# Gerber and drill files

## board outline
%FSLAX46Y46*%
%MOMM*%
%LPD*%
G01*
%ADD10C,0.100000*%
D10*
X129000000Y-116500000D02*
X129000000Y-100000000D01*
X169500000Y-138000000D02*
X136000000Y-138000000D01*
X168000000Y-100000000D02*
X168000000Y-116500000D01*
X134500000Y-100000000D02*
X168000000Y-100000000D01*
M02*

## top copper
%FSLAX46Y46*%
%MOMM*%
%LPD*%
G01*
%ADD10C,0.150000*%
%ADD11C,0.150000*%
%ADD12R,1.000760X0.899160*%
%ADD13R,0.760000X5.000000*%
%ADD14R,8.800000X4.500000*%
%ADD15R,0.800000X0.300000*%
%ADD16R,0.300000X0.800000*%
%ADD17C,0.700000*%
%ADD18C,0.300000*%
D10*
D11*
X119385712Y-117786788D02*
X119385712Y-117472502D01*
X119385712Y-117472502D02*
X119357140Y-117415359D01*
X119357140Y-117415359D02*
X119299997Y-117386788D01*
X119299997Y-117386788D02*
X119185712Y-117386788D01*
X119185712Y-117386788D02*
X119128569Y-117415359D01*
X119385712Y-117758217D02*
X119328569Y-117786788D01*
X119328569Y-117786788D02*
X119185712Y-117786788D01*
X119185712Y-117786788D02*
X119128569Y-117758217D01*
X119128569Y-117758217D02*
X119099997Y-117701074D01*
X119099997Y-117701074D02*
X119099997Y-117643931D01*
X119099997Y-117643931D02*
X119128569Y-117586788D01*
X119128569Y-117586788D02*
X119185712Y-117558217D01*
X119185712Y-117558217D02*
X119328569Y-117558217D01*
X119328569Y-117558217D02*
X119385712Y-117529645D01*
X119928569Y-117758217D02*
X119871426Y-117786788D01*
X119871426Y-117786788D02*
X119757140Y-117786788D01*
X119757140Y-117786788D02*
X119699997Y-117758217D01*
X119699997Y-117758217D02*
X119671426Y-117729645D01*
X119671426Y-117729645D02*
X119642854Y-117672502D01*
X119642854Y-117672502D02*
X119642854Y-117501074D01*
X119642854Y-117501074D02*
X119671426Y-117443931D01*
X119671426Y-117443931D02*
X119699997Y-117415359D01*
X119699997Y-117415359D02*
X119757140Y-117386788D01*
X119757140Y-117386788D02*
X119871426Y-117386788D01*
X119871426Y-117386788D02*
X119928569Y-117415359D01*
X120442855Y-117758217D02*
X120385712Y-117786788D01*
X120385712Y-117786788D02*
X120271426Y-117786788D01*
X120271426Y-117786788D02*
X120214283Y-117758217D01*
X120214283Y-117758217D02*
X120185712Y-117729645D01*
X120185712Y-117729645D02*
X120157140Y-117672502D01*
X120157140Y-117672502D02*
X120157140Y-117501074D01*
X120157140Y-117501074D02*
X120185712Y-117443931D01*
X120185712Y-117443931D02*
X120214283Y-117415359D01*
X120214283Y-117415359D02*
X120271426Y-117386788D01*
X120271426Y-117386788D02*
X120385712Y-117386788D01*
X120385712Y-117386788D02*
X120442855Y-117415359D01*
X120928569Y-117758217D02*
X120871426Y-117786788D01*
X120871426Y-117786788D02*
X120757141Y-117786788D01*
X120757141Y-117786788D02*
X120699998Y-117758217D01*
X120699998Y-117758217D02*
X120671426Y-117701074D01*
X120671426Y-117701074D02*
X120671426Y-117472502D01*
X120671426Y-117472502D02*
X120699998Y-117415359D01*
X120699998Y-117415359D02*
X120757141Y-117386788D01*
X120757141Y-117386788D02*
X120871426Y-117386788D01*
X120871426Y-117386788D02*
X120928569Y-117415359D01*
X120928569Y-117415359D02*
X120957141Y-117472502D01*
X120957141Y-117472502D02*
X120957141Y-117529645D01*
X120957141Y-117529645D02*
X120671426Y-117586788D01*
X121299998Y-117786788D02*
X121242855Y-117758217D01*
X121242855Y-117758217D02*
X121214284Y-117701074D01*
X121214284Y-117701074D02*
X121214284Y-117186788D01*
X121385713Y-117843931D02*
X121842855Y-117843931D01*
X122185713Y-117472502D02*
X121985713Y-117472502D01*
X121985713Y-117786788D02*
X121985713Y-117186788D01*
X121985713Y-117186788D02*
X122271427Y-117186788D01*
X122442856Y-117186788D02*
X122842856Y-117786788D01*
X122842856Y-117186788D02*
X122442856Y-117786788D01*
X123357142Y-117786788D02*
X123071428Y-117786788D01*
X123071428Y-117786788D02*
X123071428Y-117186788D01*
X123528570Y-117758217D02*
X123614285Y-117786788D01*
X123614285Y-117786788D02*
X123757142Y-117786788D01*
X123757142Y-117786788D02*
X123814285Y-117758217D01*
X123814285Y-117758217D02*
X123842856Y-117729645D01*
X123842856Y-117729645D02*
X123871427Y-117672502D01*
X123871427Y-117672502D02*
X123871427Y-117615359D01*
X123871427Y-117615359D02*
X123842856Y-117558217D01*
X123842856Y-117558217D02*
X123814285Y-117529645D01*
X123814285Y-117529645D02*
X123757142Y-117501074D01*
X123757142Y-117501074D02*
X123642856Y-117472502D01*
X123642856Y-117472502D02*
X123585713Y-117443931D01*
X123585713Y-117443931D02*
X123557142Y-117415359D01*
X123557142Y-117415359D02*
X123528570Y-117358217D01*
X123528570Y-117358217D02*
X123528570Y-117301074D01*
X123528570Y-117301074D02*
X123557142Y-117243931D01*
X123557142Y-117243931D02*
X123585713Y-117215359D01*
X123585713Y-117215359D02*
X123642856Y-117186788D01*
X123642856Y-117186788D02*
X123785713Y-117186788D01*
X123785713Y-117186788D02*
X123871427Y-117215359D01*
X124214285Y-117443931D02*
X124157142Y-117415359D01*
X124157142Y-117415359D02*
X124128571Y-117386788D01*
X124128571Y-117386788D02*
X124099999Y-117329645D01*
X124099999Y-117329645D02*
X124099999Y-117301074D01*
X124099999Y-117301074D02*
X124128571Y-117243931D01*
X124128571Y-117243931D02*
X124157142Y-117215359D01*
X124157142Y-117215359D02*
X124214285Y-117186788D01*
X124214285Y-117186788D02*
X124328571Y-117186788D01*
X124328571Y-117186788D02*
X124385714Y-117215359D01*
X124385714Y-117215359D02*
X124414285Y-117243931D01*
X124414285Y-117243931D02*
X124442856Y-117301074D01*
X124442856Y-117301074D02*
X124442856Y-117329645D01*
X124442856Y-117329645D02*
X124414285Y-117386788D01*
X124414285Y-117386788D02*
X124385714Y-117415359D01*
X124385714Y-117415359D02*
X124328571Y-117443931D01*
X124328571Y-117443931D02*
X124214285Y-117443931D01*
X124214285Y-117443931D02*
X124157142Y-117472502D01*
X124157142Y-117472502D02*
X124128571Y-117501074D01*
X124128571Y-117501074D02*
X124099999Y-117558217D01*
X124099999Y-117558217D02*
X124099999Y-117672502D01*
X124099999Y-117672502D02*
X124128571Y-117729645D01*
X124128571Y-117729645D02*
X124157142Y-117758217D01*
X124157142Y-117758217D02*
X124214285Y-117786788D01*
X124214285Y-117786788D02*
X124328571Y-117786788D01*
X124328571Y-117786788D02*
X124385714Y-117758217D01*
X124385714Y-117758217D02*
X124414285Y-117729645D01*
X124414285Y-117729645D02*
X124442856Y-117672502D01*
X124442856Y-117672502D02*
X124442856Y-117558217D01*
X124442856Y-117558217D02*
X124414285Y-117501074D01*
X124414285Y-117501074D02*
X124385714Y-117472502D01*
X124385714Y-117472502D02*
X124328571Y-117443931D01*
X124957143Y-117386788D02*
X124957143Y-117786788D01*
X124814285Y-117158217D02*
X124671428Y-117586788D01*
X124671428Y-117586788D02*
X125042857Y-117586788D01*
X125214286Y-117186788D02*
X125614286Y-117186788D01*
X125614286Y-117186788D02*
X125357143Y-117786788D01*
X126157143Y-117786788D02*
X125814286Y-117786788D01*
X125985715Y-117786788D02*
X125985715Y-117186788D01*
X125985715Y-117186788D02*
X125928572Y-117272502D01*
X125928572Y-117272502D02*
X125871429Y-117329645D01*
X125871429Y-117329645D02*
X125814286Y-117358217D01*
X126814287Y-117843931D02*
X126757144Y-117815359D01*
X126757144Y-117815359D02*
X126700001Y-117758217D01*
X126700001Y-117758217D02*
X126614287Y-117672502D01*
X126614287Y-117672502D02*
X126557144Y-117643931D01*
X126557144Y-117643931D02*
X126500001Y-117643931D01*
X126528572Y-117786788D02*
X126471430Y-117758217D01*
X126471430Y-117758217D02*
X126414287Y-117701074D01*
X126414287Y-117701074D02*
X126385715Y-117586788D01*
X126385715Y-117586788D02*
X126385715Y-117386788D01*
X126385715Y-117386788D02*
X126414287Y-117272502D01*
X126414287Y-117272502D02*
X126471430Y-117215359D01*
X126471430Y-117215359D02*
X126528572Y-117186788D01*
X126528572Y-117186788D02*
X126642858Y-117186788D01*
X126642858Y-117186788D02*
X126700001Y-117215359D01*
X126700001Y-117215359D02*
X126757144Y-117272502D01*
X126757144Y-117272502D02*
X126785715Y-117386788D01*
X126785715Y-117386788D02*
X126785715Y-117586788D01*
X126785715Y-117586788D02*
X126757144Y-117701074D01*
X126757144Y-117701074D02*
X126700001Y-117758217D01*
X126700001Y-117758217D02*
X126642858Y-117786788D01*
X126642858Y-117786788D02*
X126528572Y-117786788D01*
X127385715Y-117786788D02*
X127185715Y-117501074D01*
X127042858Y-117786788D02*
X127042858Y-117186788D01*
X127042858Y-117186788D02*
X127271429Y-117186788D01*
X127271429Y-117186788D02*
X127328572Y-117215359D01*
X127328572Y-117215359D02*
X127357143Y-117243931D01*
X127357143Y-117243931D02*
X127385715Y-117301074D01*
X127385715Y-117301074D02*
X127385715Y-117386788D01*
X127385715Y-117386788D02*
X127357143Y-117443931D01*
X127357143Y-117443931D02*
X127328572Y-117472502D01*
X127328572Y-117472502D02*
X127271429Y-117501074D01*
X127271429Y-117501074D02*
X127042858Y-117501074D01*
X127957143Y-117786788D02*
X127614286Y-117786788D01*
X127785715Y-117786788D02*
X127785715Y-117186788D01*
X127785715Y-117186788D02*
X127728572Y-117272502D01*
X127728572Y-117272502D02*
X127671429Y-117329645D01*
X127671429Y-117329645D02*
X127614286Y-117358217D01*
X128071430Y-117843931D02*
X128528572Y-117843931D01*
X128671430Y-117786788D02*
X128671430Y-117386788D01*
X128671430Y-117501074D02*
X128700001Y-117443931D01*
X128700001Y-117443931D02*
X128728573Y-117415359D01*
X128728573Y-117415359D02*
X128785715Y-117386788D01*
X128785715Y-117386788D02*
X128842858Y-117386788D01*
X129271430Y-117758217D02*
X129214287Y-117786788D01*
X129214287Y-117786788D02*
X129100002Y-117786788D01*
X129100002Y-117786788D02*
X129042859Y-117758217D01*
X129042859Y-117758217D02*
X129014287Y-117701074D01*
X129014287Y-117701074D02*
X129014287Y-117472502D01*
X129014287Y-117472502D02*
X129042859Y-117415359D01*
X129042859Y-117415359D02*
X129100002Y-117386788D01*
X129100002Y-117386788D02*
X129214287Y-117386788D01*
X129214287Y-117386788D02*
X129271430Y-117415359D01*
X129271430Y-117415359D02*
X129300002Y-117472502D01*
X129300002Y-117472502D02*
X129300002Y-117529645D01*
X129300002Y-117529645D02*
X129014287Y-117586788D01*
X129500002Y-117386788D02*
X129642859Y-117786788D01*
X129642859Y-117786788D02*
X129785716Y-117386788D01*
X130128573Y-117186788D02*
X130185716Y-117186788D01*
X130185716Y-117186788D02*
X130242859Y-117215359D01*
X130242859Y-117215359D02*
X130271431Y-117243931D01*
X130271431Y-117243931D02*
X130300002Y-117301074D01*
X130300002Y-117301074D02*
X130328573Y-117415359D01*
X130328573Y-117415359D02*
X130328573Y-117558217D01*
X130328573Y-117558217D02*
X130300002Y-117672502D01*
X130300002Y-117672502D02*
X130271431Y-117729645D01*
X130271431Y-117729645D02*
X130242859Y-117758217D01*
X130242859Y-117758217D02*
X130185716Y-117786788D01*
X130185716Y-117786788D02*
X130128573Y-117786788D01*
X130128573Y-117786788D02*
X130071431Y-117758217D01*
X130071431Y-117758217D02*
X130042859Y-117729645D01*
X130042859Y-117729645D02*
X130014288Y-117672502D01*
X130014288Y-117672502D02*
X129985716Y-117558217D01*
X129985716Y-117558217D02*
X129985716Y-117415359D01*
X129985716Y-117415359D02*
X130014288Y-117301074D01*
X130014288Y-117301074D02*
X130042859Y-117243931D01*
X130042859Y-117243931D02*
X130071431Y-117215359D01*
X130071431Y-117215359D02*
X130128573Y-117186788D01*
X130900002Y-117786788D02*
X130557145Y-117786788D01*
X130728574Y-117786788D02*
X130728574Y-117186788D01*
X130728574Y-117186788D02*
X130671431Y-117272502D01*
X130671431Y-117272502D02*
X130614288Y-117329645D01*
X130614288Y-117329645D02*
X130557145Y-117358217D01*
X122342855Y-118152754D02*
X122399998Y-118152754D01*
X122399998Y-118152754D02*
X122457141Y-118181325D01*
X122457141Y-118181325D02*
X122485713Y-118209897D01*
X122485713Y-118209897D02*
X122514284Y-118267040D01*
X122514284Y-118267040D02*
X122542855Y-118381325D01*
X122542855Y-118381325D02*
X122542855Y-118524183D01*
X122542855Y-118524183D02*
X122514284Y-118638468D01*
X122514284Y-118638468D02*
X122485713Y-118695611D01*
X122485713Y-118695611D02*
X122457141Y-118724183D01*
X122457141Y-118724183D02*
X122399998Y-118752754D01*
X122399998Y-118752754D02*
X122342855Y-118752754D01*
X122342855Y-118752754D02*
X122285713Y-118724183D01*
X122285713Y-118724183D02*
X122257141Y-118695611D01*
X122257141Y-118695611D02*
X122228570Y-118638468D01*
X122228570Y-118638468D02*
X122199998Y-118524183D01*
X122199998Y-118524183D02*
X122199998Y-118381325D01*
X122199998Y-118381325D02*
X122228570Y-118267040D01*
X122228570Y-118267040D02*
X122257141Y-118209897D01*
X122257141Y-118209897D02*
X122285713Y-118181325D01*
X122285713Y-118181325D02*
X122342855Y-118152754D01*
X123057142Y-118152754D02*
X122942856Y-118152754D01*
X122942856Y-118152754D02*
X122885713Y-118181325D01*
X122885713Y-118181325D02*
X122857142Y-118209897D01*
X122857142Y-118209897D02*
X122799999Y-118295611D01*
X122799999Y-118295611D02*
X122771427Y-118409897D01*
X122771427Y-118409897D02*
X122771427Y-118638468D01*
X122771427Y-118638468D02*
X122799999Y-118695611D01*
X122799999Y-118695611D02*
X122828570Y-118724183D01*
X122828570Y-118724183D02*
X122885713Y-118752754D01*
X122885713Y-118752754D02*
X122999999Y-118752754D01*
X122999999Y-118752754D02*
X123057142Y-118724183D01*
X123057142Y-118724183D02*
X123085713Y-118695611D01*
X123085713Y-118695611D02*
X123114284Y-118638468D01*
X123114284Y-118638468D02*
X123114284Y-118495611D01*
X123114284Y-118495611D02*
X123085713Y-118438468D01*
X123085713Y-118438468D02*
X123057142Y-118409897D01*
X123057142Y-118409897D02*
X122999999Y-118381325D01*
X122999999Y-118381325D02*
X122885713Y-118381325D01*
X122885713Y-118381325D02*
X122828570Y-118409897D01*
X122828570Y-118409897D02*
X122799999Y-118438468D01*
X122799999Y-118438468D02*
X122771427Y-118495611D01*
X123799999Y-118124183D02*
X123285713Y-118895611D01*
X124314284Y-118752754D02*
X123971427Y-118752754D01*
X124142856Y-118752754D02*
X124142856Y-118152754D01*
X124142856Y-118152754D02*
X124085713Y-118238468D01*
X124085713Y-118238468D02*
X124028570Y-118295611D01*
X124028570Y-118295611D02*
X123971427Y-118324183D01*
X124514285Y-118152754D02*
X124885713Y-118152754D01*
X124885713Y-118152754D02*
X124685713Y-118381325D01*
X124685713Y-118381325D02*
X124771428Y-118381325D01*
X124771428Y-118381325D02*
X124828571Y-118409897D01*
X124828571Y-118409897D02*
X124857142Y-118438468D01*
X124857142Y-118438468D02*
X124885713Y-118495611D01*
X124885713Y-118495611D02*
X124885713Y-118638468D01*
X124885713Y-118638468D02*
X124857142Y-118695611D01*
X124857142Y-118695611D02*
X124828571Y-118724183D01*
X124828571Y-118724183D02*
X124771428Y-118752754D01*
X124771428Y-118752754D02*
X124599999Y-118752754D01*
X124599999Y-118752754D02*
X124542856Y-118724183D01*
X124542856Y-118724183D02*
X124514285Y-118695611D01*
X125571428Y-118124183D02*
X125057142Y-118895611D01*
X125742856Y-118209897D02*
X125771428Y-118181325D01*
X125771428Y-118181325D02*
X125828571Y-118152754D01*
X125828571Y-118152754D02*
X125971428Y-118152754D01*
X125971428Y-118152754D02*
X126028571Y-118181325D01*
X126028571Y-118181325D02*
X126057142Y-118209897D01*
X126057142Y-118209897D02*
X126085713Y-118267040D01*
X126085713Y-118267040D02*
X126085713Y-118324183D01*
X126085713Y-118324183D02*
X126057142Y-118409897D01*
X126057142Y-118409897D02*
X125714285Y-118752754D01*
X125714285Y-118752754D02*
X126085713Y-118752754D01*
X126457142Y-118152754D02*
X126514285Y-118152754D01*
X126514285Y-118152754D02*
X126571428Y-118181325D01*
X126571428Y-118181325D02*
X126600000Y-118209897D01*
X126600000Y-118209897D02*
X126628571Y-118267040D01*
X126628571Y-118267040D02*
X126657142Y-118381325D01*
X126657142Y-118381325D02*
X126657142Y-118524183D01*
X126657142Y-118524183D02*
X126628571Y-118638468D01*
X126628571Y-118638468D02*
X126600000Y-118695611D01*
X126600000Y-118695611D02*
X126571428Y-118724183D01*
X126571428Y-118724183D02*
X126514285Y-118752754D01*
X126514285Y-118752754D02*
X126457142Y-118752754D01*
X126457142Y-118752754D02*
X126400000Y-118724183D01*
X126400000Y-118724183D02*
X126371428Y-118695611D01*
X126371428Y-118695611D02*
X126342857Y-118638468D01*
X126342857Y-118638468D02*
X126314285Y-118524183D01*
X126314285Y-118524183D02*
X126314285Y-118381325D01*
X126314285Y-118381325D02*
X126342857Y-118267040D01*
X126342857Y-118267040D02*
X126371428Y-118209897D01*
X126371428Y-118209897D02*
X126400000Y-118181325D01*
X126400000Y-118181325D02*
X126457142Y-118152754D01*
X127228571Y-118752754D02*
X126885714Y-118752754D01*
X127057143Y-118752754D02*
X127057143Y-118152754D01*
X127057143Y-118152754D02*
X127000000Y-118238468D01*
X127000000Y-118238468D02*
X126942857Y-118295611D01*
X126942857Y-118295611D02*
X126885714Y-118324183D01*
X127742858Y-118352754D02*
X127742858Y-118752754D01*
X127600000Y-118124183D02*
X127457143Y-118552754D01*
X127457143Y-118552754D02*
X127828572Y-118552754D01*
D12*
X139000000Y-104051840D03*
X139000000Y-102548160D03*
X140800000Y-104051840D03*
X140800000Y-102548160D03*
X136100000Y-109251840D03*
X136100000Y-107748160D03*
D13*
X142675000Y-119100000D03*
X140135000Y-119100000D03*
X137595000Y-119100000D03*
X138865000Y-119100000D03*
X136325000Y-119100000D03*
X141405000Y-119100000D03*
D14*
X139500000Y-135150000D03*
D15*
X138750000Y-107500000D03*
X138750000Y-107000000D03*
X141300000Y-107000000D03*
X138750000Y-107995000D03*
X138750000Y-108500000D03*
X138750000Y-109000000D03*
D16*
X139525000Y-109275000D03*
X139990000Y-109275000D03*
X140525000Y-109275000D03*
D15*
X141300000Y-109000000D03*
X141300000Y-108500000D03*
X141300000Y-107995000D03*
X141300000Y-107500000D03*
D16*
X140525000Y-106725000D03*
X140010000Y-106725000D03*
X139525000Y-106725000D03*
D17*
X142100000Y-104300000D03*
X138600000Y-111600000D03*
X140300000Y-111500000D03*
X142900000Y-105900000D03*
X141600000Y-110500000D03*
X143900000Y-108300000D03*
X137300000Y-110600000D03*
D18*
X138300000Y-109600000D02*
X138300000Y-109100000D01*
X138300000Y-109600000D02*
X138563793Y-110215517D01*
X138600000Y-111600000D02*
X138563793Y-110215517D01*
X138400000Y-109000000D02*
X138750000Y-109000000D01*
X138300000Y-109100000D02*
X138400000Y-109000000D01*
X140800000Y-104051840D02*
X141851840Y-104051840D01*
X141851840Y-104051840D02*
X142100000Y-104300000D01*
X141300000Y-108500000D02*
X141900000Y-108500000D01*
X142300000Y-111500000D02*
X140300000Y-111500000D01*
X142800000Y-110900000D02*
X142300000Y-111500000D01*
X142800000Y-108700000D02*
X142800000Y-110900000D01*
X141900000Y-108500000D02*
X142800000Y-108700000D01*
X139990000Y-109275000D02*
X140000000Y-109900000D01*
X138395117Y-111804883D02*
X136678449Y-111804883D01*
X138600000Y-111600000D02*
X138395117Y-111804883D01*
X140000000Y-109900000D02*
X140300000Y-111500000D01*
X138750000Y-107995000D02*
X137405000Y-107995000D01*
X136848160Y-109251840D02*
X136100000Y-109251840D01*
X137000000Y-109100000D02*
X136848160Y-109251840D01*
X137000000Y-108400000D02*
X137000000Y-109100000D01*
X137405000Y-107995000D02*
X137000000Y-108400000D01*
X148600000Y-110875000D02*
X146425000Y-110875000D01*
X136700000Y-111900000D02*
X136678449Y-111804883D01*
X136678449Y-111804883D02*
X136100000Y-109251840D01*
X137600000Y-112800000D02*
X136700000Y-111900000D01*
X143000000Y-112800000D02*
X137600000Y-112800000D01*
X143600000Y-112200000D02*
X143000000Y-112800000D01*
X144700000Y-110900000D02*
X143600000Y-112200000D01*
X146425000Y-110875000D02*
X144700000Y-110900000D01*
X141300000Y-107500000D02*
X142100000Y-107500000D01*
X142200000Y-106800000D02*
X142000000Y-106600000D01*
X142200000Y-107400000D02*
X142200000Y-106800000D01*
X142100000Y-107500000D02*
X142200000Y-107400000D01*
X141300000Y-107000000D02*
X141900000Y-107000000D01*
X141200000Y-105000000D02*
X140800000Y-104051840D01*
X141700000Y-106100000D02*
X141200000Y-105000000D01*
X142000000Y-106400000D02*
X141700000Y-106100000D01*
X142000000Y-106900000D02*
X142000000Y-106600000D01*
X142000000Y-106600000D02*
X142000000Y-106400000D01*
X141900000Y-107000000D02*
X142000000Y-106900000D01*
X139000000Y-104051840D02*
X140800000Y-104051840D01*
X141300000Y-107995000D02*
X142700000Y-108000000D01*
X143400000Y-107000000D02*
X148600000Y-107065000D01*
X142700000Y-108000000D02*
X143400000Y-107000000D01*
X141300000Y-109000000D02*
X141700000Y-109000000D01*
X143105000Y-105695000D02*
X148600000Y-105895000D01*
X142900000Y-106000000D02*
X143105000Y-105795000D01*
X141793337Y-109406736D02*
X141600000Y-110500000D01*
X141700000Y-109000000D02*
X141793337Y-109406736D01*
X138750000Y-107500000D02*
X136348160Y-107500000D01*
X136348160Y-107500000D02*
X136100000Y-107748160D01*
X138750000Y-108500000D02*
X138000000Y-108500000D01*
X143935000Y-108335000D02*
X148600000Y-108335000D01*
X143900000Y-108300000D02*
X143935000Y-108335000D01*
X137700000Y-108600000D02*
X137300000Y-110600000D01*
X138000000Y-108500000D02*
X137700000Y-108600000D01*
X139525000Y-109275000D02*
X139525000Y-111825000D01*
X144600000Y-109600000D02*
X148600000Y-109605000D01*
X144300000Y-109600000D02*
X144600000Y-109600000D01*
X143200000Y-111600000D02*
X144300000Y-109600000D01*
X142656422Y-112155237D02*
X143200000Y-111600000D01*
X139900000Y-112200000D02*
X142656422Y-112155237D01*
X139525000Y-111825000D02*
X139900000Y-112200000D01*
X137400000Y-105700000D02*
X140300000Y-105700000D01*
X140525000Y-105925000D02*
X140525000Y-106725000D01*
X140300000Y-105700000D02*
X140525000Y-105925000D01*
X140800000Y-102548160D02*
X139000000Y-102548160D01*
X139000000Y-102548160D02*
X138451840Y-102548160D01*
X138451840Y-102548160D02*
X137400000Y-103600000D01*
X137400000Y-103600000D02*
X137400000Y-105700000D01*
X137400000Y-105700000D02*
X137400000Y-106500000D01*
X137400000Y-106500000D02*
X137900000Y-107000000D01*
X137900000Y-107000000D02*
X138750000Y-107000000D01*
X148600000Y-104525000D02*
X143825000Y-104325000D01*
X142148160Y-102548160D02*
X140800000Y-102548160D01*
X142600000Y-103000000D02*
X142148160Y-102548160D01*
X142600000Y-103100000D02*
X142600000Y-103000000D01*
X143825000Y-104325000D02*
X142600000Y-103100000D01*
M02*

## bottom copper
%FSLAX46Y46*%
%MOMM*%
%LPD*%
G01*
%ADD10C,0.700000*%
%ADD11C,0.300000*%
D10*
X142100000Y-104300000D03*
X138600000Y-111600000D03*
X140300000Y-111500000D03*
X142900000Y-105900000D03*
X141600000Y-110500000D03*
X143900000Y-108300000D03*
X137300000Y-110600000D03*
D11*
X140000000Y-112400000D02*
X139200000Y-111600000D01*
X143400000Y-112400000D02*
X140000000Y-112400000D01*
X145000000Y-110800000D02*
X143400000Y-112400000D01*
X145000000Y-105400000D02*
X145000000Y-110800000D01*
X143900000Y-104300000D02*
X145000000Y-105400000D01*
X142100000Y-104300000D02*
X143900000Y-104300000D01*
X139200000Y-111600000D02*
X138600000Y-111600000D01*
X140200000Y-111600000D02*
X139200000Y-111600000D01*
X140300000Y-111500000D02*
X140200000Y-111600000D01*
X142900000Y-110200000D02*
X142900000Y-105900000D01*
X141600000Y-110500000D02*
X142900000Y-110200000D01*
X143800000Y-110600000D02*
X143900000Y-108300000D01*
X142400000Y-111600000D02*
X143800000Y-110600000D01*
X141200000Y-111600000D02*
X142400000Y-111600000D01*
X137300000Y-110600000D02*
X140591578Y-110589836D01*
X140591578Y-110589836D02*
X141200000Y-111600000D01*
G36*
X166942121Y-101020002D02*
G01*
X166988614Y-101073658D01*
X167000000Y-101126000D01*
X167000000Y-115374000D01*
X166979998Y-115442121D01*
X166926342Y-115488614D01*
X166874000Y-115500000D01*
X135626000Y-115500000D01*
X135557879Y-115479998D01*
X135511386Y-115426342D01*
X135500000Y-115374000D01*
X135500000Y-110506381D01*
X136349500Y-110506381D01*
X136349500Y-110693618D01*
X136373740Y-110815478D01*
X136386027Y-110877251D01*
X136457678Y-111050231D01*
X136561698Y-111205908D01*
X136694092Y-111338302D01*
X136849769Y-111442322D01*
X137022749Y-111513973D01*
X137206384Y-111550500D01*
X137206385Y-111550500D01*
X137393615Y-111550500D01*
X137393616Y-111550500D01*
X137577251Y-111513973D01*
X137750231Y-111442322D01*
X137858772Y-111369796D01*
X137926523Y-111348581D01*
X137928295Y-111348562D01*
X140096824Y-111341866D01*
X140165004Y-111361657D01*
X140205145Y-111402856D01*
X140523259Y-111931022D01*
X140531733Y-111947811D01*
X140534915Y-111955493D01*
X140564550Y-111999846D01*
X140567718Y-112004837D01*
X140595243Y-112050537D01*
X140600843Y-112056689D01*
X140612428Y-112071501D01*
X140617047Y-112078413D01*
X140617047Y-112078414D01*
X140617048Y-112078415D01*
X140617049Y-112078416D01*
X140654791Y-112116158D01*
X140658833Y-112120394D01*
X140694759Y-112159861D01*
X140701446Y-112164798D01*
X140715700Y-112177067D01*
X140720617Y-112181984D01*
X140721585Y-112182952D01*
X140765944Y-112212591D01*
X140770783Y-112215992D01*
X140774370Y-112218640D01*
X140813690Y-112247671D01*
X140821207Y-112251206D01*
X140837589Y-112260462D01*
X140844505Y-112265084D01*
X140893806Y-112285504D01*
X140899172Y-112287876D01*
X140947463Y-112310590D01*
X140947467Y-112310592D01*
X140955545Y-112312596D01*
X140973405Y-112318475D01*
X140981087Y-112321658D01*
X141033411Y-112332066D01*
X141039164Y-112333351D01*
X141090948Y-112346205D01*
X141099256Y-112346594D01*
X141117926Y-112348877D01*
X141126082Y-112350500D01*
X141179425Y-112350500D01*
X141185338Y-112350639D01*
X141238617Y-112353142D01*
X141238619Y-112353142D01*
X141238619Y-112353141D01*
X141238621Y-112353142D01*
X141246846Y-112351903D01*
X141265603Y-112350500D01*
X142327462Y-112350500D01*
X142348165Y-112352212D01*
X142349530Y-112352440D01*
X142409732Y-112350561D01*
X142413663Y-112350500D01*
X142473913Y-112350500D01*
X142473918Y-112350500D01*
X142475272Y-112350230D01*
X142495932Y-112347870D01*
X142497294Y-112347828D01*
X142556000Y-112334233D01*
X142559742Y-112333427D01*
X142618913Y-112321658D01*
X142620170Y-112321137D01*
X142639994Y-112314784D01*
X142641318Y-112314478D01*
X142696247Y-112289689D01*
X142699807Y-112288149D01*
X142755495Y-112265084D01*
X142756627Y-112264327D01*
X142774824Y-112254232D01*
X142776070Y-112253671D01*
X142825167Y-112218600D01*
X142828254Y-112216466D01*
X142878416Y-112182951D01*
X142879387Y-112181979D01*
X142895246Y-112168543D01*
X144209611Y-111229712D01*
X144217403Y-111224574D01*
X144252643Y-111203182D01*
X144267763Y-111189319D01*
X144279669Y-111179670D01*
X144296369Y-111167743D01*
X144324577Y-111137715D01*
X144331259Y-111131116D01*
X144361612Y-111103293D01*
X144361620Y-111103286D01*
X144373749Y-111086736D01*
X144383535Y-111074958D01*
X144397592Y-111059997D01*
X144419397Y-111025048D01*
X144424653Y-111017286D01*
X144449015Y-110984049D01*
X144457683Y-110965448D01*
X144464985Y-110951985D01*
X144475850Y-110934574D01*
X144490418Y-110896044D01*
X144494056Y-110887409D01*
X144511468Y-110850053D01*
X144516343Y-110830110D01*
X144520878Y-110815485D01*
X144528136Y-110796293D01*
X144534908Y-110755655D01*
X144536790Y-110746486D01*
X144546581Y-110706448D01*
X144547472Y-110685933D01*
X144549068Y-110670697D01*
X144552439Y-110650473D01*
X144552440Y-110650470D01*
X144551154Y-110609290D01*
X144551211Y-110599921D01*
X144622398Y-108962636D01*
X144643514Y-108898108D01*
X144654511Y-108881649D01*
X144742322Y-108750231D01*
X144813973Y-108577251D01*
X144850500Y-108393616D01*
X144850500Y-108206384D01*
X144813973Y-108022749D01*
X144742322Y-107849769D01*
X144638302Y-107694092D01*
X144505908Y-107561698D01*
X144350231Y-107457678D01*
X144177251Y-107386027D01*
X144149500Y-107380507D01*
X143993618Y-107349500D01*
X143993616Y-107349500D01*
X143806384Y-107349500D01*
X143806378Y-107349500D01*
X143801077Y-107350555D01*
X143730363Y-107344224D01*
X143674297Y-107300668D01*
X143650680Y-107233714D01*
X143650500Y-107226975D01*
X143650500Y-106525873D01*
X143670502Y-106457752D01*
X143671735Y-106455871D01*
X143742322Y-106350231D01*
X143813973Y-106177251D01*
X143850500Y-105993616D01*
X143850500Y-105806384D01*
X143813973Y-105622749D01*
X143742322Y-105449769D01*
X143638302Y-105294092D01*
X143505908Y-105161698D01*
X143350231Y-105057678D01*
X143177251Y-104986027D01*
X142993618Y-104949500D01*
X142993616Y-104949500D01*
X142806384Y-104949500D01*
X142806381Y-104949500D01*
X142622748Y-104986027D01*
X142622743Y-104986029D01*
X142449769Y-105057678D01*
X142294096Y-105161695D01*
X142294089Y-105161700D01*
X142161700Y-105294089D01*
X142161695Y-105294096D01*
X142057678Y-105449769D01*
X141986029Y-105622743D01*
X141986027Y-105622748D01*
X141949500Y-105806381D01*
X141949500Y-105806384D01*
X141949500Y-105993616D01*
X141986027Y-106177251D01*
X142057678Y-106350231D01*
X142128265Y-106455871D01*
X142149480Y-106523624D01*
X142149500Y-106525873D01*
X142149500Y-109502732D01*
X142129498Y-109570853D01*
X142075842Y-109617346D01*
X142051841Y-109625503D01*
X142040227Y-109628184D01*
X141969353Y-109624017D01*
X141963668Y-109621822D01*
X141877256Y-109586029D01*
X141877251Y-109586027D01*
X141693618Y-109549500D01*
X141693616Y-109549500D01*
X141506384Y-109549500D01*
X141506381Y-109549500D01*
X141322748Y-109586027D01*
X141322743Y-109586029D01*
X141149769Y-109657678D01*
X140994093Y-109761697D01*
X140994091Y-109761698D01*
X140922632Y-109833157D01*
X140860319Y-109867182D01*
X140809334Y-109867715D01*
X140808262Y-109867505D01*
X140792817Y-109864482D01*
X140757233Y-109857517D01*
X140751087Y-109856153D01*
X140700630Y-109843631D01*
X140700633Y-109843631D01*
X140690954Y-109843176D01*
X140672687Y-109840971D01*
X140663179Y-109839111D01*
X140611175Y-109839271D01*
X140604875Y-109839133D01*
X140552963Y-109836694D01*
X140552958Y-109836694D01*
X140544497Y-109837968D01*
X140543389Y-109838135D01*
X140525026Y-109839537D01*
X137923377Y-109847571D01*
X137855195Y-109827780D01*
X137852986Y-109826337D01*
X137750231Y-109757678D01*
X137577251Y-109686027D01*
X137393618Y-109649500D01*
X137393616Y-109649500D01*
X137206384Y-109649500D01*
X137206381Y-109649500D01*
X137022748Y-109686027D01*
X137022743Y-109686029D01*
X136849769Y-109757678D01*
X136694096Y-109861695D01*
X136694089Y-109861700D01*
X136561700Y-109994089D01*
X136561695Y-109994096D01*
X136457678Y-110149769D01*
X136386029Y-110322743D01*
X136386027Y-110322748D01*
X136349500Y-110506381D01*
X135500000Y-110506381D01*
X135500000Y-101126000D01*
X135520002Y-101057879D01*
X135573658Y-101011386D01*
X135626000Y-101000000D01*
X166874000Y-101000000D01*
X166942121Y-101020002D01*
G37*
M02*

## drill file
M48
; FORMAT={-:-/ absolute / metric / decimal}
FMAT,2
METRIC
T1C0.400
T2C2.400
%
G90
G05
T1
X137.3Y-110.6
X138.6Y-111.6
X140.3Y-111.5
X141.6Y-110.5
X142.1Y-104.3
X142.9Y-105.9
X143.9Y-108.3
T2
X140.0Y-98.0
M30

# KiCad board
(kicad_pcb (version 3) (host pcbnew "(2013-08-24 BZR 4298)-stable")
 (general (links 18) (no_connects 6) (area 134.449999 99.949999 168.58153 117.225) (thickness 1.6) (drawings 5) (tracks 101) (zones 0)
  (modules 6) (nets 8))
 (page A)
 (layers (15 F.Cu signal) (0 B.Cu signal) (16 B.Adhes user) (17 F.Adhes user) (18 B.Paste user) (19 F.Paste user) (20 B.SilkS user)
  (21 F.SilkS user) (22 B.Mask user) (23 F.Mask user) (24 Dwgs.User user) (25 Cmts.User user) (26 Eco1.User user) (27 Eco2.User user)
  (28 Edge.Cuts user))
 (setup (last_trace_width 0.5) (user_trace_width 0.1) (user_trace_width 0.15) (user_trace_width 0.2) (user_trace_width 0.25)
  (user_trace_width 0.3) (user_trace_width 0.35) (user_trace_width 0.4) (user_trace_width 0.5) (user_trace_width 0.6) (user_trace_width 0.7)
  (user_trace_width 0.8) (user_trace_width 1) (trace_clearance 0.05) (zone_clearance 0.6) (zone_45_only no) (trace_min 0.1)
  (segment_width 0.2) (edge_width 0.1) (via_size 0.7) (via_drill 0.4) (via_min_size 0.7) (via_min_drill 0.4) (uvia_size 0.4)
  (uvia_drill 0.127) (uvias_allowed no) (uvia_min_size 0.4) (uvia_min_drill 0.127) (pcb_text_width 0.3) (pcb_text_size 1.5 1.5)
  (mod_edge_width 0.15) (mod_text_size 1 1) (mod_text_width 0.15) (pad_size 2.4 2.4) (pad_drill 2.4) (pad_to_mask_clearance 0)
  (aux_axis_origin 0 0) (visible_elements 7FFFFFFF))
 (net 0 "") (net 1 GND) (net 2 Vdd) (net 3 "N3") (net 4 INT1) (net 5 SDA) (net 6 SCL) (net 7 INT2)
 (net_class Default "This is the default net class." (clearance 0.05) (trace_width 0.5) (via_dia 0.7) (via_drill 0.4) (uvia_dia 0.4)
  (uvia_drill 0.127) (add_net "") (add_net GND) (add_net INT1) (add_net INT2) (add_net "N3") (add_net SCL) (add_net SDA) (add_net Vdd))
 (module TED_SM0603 (layer F.Cu) (at 139 103.3 270)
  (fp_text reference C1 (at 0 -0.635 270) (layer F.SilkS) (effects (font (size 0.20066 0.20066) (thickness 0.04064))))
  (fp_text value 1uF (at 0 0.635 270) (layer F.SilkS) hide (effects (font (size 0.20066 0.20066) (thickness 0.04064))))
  (pad 2 smd rect (at 0.75184 0 270) (size 0.89916 1.00076) (layers F.Cu F.Paste F.Mask) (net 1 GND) (clearance 0.1))
  (pad 1 smd rect (at -0.75184 0 270) (size 0.89916 1.00076) (layers F.Cu F.Paste F.Mask) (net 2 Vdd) (clearance 0.1)))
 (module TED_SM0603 (layer F.Cu) (at 140.8 103.3 270)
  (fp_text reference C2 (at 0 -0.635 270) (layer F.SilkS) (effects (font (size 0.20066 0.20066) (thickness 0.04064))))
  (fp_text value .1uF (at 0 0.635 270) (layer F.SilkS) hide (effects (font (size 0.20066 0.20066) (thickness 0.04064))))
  (pad 2 smd rect (at 0.75184 0 270) (size 0.89916 1.00076) (layers F.Cu F.Paste F.Mask) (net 1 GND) (clearance 0.1))
  (pad 1 smd rect (at -0.75184 0 270) (size 0.89916 1.00076) (layers F.Cu F.Paste F.Mask) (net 2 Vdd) (clearance 0.1)))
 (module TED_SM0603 (layer F.Cu) (at 136.1 108.5 270)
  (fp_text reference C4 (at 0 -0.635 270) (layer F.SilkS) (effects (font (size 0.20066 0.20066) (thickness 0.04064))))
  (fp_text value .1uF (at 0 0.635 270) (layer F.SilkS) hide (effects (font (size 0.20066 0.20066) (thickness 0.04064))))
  (pad 2 smd rect (at 0.75184 0 270) (size 0.89916 1.00076) (layers F.Cu F.Paste F.Mask) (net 1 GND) (clearance 0.1))
  (pad 1 smd rect (at -0.75184 0 270) (size 0.89916 1.00076) (layers F.Cu F.Paste F.Mask) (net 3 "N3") (clearance 0.1)))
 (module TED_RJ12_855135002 (layer F.Cu) (at 139.5 127 180)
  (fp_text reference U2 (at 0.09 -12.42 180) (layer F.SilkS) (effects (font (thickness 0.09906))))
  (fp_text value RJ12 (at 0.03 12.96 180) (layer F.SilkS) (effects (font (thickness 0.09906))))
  (pad 6 smd rect (at -3.175 7.9 180) (size 0.76 5) (layers F.Cu F.Paste F.Mask) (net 2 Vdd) (clearance 0.2))
  (pad 4 smd rect (at -0.635 7.9 180) (size 0.76 5) (layers F.Cu F.Paste F.Mask) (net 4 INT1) (clearance 0.2))
  (pad 2 smd rect (at 1.905 7.9 180) (size 0.76 5) (layers F.Cu F.Paste F.Mask) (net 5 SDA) (clearance 0.2))
  (pad 3 smd rect (at 0.635 7.9 180) (size 0.76 5) (layers F.Cu F.Paste F.Mask) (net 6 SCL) (clearance 0.2))
  (pad 1 smd rect (at 3.175 7.9 180) (size 0.76 5) (layers F.Cu F.Paste F.Mask) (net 1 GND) (clearance 0.2))
  (pad 5 smd rect (at -1.905 7.9 180) (size 0.76 5) (layers F.Cu F.Paste F.Mask) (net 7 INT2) (clearance 0.2))
  (pad PAD smd rect (at 0 -8.15 180) (size 8.8 4.5) (layers F.Cu F.Paste F.Mask)))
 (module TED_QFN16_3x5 (layer F.Cu) (at 140.025 108) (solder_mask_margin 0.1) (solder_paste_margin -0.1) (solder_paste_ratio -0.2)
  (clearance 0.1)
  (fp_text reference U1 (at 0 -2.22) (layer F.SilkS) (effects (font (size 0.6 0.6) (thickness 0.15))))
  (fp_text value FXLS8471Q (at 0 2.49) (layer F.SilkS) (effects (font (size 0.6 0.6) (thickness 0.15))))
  (pad 2 smd rect (at -1.275 -0.5) (size 0.8 0.3) (layers F.Cu F.Paste F.Mask) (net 3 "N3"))
  (pad 1 smd rect (at -1.275 -1) (size 0.8 0.3) (layers F.Cu F.Paste F.Mask) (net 2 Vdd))
  (pad 13 smd rect (at 1.275 -1) (size 0.8 0.3) (layers F.Cu F.Paste F.Mask) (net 1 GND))
  (pad 3 smd rect (at -1.275 -0.005) (size 0.8 0.3) (layers F.Cu F.Paste F.Mask) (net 1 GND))
  (pad 4 smd rect (at -1.275 0.5) (size 0.8 0.3) (layers F.Cu F.Paste F.Mask) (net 6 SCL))
  (pad 5 smd rect (at -1.275 1) (size 0.8 0.3) (layers F.Cu F.Paste F.Mask) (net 1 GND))
  (pad 6 smd rect (at -0.5 1.275) (size 0.3 0.8) (layers F.Cu F.Paste F.Mask) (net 5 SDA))
  (pad 7 smd rect (at -0.035 1.275) (size 0.3 0.8) (layers F.Cu F.Paste F.Mask) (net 1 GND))
  (pad 8 smd rect (at 0.5 1.275) (size 0.3 0.8) (layers F.Cu F.Paste F.Mask))
  (pad 9 smd rect (at 1.275 1) (size 0.8 0.3) (layers F.Cu F.Paste F.Mask) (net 7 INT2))
  (pad 10 smd rect (at 1.275 0.5) (size 0.8 0.3) (layers F.Cu F.Paste F.Mask) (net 1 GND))
  (pad 11 smd rect (at 1.275 -0.005) (size 0.8 0.3) (layers F.Cu F.Paste F.Mask) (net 4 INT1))
  (pad 12 smd rect (at 1.275 -0.5) (size 0.8 0.3) (layers F.Cu F.Paste F.Mask) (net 1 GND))
  (pad 14 smd rect (at 0.5 -1.275) (size 0.3 0.8) (layers F.Cu F.Paste F.Mask) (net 2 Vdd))
  (pad 15 smd rect (at -0.015 -1.275) (size 0.3 0.8) (layers F.Cu F.Paste F.Mask))
  (pad 16 smd rect (at -0.5 -1.275) (size 0.3 0.8) (layers F.Cu F.Paste F.Mask)))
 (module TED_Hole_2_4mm (layer F.Cu) (at 132.5 108)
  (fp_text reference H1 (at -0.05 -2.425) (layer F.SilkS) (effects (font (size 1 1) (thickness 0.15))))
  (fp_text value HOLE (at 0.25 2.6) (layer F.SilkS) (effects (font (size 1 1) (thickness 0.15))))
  (pad "" np_thru_hole circle (at 7.5 -10) (size 2.4 2.4) (drill 2.4) (layers *.Cu *.Mask F.SilkS)))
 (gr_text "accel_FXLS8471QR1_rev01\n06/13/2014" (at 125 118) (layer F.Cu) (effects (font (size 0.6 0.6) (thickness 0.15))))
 (gr_line (start 129 116.5) (end 129 100) (angle 90) (layer Edge.Cuts) (width 0.1))
 (gr_line (start 169.5 138) (end 136 138) (angle 90) (layer Edge.Cuts) (width 0.1))
 (gr_line (start 168 100) (end 168 116.5) (angle 90) (layer Edge.Cuts) (width 0.1))
 (gr_line (start 134.5 100) (end 168 100) (angle 90) (layer Edge.Cuts) (width 0.1))
 (segment (start 138.3 109.6) (end 138.3 109.1) (width 0.3) (layer F.Cu) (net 1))
 (segment (start 138.3 109.6) (end 138.563793 110.215517) (width 0.3) (layer F.Cu) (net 1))
 (segment (start 138.6 111.6) (end 138.563793 110.215517) (width 0.3) (layer F.Cu) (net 1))
 (segment (start 138.4 109) (end 138.75 109) (width 0.3) (layer F.Cu) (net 1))
 (segment (start 138.3 109.1) (end 138.4 109) (width 0.3) (layer F.Cu) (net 1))
 (segment (start 140.8 104.05184) (end 141.85184 104.05184) (width 0.3) (layer F.Cu) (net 1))
 (segment (start 140 112.4) (end 139.2 111.6) (width 0.3) (layer B.Cu) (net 1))
 (segment (start 143.4 112.4) (end 140 112.4) (width 0.3) (layer B.Cu) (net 1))
 (segment (start 145 110.8) (end 143.4 112.4) (width 0.3) (layer B.Cu) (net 1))
 (segment (start 145 105.4) (end 145 110.8) (width 0.3) (layer B.Cu) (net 1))
 (segment (start 143.9 104.3) (end 145 105.4) (width 0.3) (layer B.Cu) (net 1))
 (segment (start 142.1 104.3) (end 143.9 104.3) (width 0.3) (layer B.Cu) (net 1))
 (via (at 142.1 104.3) (size 0.7) (layers F.Cu B.Cu) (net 1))
 (segment (start 141.85184 104.05184) (end 142.1 104.3) (width 0.3) (layer F.Cu) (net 1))
 (segment (start 141.3 108.5) (end 141.9 108.5) (width 0.3) (layer F.Cu) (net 1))
 (segment (start 142.3 111.5) (end 140.3 111.5) (width 0.3) (layer F.Cu) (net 1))
 (segment (start 142.8 110.9) (end 142.3 111.5) (width 0.3) (layer F.Cu) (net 1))
 (segment (start 142.8 108.7) (end 142.8 110.9) (width 0.3) (layer F.Cu) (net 1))
 (segment (start 141.9 108.5) (end 142.8 108.7) (width 0.3) (layer F.Cu) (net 1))
 (segment (start 139.99 109.275) (end 140 109.9) (width 0.3) (layer F.Cu) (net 1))
 (segment (start 138.395117 111.804883) (end 136.678449 111.804883) (width 0.3) (layer F.Cu) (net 1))
 (segment (start 138.6 111.6) (end 138.395117 111.804883) (width 0.3) (layer F.Cu) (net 1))
 (via (at 138.6 111.6) (size 0.7) (layers F.Cu B.Cu) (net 1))
 (segment (start 139.2 111.6) (end 138.6 111.6) (width 0.3) (layer B.Cu) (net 1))
 (segment (start 140.2 111.6) (end 139.2 111.6) (width 0.3) (layer B.Cu) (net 1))
 (via (at 140.3 111.5) (size 0.7) (layers F.Cu B.Cu) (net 1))
 (segment (start 140.3 111.5) (end 140.2 111.6) (width 0.3) (layer B.Cu) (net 1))
 (segment (start 140 109.9) (end 140.3 111.5) (width 0.3) (layer F.Cu) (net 1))
 (segment (start 138.75 107.995) (end 137.405 107.995) (width 0.3) (layer F.Cu) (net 1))
 (segment (start 136.84816 109.25184) (end 136.1 109.25184) (width 0.3) (layer F.Cu) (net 1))
 (segment (start 137 109.1) (end 136.84816 109.25184) (width 0.3) (layer F.Cu) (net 1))
 (segment (start 137 108.4) (end 137 109.1) (width 0.3) (layer F.Cu) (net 1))
 (segment (start 137.405 107.995) (end 137 108.4) (width 0.3) (layer F.Cu) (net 1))
 (segment (start 148.6 110.875) (end 146.425 110.875) (width 0.3) (layer F.Cu) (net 1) (status 30))
 (segment (start 136.7 111.9) (end 136.678449 111.804883) (width 0.3) (layer F.Cu) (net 1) (status 20))
 (segment (start 136.678449 111.804883) (end 136.1 109.25184) (width 0.3) (layer F.Cu) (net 1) (status 20))
 (segment (start 137.6 112.8) (end 136.7 111.9) (width 0.3) (layer F.Cu) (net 1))
 (segment (start 143 112.8) (end 137.6 112.8) (width 0.3) (layer F.Cu) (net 1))
 (segment (start 143.6 112.2) (end 143 112.8) (width 0.3) (layer F.Cu) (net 1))
 (segment (start 144.7 110.9) (end 143.6 112.2) (width 0.3) (layer F.Cu) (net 1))
 (segment (start 146.425 110.875) (end 144.7 110.9) (width 0.3) (layer F.Cu) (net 1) (status 10))
 (segment (start 141.3 107.5) (end 142.1 107.5) (width 0.3) (layer F.Cu) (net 1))
 (segment (start 142.2 106.8) (end 142 106.6) (width 0.3) (layer F.Cu) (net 1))
 (segment (start 142.2 107.4) (end 142.2 106.8) (width 0.3) (layer F.Cu) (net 1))
 (segment (start 142.1 107.5) (end 142.2 107.4) (width 0.3) (layer F.Cu) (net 1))
 (segment (start 141.3 107) (end 141.9 107) (width 0.3) (layer F.Cu) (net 1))
 (segment (start 141.2 105) (end 140.8 104.05184) (width 0.3) (layer F.Cu) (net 1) (status 20))
 (segment (start 141.7 106.1) (end 141.2 105) (width 0.3) (layer F.Cu) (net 1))
 (segment (start 142 106.4) (end 141.7 106.1) (width 0.3) (layer F.Cu) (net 1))
 (segment (start 142 106.9) (end 142 106.6) (width 0.3) (layer F.Cu) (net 1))
 (segment (start 142 106.6) (end 142 106.4) (width 0.3) (layer F.Cu) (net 1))
 (segment (start 141.9 107) (end 142 106.9) (width 0.3) (layer F.Cu) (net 1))
 (segment (start 139 104.05184) (end 140.8 104.05184) (width 0.3) (layer F.Cu) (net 1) (status 20))
 (segment (start 141.3 107.995) (end 142.7 108) (width 0.3) (layer F.Cu) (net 4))
 (segment (start 143.4 107) (end 148.6 107.065) (width 0.3) (layer F.Cu) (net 4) (status 20))
 (segment (start 142.7 108) (end 143.4 107) (width 0.3) (layer F.Cu) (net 4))
 (segment (start 141.3 109) (end 141.7 109) (width 0.3) (layer F.Cu) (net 7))
 (segment (start 143.105 105.695) (end 148.6 105.895) (width 0.3) (layer F.Cu) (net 7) (status 20))
 (segment (start 142.9 106) (end 143.105 105.795) (width 0.3) (layer F.Cu) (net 7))
 (via (at 142.9 105.9) (size 0.7) (layers F.Cu B.Cu) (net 7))
 (segment (start 142.9 110.2) (end 142.9 105.9) (width 0.3) (layer B.Cu) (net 7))
 (segment (start 141.6 110.5) (end 142.9 110.2) (width 0.3) (layer B.Cu) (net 7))
 (via (at 141.6 110.5) (size 0.7) (layers F.Cu B.Cu) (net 7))
 (segment (start 141.793337 109.406736) (end 141.6 110.5) (width 0.3) (layer F.Cu) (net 7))
 (segment (start 141.7 109) (end 141.793337 109.406736) (width 0.3) (layer F.Cu) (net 7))
 (segment (start 138.75 107.5) (end 136.34816 107.5) (width 0.3) (layer F.Cu) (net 3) (status 20))
 (segment (start 136.34816 107.5) (end 136.1 107.74816) (width 0.3) (layer F.Cu) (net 3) (status 30))
 (segment (start 138.75 108.5) (end 138 108.5) (width 0.3) (layer F.Cu) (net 6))
 (segment (start 143.935 108.335) (end 148.6 108.335) (width 0.3) (layer F.Cu) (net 6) (status 20))
 (segment (start 143.9 108.3) (end 143.935 108.335) (width 0.3) (layer F.Cu) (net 6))
 (via (at 143.9 108.3) (size 0.7) (layers F.Cu B.Cu) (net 6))
 (segment (start 143.8 110.6) (end 143.9 108.3) (width 0.3) (layer B.Cu) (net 6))
 (segment (start 142.4 111.6) (end 143.8 110.6) (width 0.3) (layer B.Cu) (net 6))
 (segment (start 141.2 111.6) (end 142.4 111.6) (width 0.3) (layer B.Cu) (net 6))
 (segment (start 137.3 110.6) (end 140.591578 110.589836) (width 0.3) (layer B.Cu) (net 6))
 (segment (start 140.591578 110.589836) (end 141.2 111.6) (width 0.3) (layer B.Cu) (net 6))
 (via (at 137.3 110.6) (size 0.7) (layers F.Cu B.Cu) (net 6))
 (segment (start 137.7 108.6) (end 137.3 110.6) (width 0.3) (layer F.Cu) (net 6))
 (segment (start 138 108.5) (end 137.7 108.6) (width 0.3) (layer F.Cu) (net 6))
 (segment (start 139.525 109.275) (end 139.525 111.825) (width 0.3) (layer F.Cu) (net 5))
 (segment (start 144.6 109.6) (end 148.6 109.605) (width 0.3) (layer F.Cu) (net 5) (status 20))
 (segment (start 144.3 109.6) (end 144.6 109.6) (width 0.3) (layer F.Cu) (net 5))
 (segment (start 143.2 111.6) (end 144.3 109.6) (width 0.3) (layer F.Cu) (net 5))
 (segment (start 142.656422 112.155237) (end 143.2 111.6) (width 0.3) (layer F.Cu) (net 5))
 (segment (start 139.9 112.2) (end 142.656422 112.155237) (width 0.3) (layer F.Cu) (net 5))
 (segment (start 139.525 111.825) (end 139.9 112.2) (width 0.3) (layer F.Cu) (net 5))
 (segment (start 137.4 105.7) (end 140.3 105.7) (width 0.3) (layer F.Cu) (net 2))
 (segment (start 140.525 105.925) (end 140.525 106.725) (width 0.3) (layer F.Cu) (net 2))
 (segment (start 140.3 105.7) (end 140.525 105.925) (width 0.3) (layer F.Cu) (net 2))
 (segment (start 140.8 102.54816) (end 139 102.54816) (width 0.3) (layer F.Cu) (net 2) (status 10))
 (segment (start 139 102.54816) (end 138.45184 102.54816) (width 0.3) (layer F.Cu) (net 2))
 (segment (start 138.45184 102.54816) (end 137.4 103.6) (width 0.3) (layer F.Cu) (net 2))
 (segment (start 137.4 103.6) (end 137.4 105.7) (width 0.3) (layer F.Cu) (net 2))
 (segment (start 137.4 105.7) (end 137.4 106.5) (width 0.3) (layer F.Cu) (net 2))
 (segment (start 137.4 106.5) (end 137.9 107) (width 0.3) (layer F.Cu) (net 2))
 (segment (start 137.9 107) (end 138.75 107) (width 0.3) (layer F.Cu) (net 2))
 (segment (start 148.6 104.525) (end 143.825 104.325) (width 0.3) (layer F.Cu) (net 2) (status 10))
 (segment (start 142.14816 102.54816) (end 140.8 102.54816) (width 0.3) (layer F.Cu) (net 2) (status 20))
 (segment (start 142.6 103) (end 142.14816 102.54816) (width 0.3) (layer F.Cu) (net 2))
 (segment (start 142.6 103.1) (end 142.6 103) (width 0.3) (layer F.Cu) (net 2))
 (segment (start 143.825 104.325) (end 142.6 103.1) (width 0.3) (layer F.Cu) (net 2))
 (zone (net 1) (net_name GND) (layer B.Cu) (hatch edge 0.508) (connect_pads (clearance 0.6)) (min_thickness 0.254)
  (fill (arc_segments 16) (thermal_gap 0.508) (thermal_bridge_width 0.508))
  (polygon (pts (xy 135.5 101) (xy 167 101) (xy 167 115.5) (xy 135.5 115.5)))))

